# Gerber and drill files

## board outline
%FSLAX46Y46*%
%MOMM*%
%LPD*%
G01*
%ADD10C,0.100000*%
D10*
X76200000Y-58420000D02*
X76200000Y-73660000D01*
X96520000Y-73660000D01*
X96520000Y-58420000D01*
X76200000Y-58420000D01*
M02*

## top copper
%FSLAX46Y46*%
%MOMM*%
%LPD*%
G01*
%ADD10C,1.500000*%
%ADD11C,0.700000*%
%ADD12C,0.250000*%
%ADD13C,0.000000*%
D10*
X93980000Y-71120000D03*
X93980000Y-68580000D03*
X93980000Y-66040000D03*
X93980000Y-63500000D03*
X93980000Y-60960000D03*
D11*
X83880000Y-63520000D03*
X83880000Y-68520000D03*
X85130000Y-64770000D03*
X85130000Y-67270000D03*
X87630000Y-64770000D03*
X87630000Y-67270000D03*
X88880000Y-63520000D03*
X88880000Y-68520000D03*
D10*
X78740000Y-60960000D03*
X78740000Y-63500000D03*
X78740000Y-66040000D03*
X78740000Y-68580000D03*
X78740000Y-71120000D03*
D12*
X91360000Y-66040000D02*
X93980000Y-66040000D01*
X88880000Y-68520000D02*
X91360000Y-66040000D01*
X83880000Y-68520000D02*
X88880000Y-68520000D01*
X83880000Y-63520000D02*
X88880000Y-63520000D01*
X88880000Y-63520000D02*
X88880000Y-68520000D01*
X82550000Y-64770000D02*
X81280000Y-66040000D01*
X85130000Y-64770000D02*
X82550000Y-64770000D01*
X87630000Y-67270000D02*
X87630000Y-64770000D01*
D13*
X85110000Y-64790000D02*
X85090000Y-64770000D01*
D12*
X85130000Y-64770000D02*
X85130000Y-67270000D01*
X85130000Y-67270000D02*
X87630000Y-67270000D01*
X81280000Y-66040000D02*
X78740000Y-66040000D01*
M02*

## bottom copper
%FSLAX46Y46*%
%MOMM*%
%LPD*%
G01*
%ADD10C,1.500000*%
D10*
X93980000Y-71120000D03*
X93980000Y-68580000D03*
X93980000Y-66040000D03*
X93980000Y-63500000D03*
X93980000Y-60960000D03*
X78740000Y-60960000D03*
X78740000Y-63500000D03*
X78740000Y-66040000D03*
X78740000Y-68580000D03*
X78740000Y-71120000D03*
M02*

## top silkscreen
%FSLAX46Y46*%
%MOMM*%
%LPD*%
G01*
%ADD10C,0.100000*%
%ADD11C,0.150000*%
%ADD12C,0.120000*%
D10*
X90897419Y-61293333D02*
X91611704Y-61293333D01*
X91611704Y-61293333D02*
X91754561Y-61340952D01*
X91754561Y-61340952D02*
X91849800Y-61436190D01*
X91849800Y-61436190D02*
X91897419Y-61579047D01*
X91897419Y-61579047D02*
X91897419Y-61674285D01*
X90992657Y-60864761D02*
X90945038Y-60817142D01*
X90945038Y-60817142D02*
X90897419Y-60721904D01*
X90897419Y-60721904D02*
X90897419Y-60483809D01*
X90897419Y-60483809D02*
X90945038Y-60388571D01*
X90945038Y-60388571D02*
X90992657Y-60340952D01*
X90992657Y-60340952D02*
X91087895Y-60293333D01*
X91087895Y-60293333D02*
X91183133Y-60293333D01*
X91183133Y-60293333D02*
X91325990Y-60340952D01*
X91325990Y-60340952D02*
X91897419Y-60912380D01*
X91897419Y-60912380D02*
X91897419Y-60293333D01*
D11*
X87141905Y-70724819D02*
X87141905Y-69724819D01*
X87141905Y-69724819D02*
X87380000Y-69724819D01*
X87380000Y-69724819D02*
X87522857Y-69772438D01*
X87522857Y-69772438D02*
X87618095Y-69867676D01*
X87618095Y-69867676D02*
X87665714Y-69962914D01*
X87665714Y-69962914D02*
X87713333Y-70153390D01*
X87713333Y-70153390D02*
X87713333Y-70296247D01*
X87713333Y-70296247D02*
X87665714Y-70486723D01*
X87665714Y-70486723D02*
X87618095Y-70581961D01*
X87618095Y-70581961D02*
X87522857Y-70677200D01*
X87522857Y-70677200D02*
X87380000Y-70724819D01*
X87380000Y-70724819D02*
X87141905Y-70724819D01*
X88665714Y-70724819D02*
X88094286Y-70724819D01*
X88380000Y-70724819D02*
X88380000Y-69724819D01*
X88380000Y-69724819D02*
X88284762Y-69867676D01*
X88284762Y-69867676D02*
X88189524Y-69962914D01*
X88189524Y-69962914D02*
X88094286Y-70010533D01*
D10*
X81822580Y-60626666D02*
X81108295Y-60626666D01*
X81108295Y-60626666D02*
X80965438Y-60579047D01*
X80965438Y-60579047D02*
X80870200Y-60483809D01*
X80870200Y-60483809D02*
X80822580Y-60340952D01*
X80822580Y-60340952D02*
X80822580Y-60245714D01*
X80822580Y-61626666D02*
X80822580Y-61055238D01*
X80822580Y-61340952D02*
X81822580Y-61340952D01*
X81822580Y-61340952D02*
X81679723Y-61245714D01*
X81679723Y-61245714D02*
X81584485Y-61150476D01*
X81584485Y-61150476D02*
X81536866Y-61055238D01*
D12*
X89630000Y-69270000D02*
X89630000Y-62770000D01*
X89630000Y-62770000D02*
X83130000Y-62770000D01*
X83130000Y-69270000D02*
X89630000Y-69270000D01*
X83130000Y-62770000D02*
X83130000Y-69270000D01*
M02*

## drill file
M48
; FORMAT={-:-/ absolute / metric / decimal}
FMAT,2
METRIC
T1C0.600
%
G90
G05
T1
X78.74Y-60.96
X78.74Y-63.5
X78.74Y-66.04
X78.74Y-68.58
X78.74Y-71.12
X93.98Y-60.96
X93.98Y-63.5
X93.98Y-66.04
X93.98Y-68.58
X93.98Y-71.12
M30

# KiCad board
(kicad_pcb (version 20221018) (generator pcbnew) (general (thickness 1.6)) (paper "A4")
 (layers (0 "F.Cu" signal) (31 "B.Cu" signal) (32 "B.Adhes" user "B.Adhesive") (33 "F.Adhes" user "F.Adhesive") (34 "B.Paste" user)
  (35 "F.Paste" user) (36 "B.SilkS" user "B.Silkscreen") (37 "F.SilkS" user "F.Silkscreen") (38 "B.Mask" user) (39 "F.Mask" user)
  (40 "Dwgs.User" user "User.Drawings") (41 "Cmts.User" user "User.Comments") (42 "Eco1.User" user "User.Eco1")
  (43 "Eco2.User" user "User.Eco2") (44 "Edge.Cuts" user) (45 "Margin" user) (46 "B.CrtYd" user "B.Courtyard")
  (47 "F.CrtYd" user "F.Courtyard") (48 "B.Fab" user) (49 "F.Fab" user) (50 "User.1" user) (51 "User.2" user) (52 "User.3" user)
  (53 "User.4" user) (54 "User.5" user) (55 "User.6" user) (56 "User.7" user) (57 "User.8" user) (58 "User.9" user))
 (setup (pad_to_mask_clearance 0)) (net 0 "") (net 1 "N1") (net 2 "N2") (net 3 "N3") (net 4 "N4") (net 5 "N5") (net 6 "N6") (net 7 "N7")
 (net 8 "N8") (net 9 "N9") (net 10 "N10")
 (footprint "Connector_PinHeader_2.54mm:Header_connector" (layer "F.Cu") (at 93.98 66.04 90)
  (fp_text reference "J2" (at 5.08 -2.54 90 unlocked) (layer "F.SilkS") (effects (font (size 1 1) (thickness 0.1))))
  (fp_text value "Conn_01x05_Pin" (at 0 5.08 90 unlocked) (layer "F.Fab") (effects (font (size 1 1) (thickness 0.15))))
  (pad "1" thru_hole circle (at -5.08 0) (size 1.5 1.5) (drill 0.6) (layers "*.Cu" "*.Mask") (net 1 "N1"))
  (pad "2" thru_hole circle (at -2.54 0) (size 1.5 1.5) (drill 0.6) (layers "*.Cu" "*.Mask") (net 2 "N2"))
  (pad "3" thru_hole circle (at 0 0) (size 1.5 1.5) (drill 0.6) (layers "*.Cu" "*.Mask") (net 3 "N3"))
  (pad "4" thru_hole circle (at 2.54 0) (size 1.5 1.5) (drill 0.6) (layers "*.Cu" "*.Mask") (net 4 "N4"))
  (pad "5" thru_hole circle (at 5.08 0) (size 1.5 1.5) (drill 0.6) (layers "*.Cu" "*.Mask") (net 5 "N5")))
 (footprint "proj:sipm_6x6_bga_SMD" (layer "F.Cu") (at 83.88 63.52 180)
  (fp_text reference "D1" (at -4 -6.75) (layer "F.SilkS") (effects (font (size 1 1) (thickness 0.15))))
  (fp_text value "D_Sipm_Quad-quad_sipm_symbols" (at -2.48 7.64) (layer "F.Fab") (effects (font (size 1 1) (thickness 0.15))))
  (fp_line (start -5.75 -5.75) (end -5.75 0.75) (stroke (width 0.12) (type solid)) (layer "F.SilkS"))
  (fp_line (start -5.75 0.75) (end 0.75 0.75) (stroke (width 0.12) (type solid)) (layer "F.SilkS"))
  (fp_line (start 0.75 -5.75) (end -5.75 -5.75) (stroke (width 0.12) (type solid)) (layer "F.SilkS"))
  (fp_line (start 0.75 0.75) (end 0.75 -5.75) (stroke (width 0.12) (type solid)) (layer "F.SilkS"))
  (pad "A1" smd circle (at 0 0 180) (size 0.7 0.7) (layers "F.Cu" "F.Paste" "F.Mask") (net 3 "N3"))
  (pad "A4" smd circle (at 0 -5 180) (size 0.7 0.7) (layers "F.Cu" "F.Paste" "F.Mask") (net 3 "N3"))
  (pad "B2" smd circle (at -1.25 -1.25 180) (size 0.7 0.7) (layers "F.Cu" "F.Paste" "F.Mask") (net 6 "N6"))
  (pad "B3" smd circle (at -1.25 -3.75 180) (size 0.7 0.7) (layers "F.Cu" "F.Paste" "F.Mask") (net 6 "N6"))
  (pad "C2" smd circle (at -3.75 -1.25 180) (size 0.7 0.7) (layers "F.Cu" "F.Paste" "F.Mask") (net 6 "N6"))
  (pad "C3" smd circle (at -3.75 -3.75 180) (size 0.7 0.7) (layers "F.Cu" "F.Paste" "F.Mask") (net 6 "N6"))
  (pad "D1" smd circle (at -5 0 180) (size 0.7 0.7) (layers "F.Cu" "F.Paste" "F.Mask") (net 3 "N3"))
  (pad "D4" smd circle (at -5 -5 180) (size 0.7 0.7) (layers "F.Cu" "F.Paste" "F.Mask") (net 3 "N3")))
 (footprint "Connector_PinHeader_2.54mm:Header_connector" (layer "F.Cu") (at 78.74 66.04 -90)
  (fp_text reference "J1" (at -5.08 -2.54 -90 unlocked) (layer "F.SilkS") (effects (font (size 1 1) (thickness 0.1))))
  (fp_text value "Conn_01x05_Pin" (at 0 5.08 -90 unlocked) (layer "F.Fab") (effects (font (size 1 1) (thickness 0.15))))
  (pad "1" thru_hole circle (at -5.08 0 180) (size 1.5 1.5) (drill 0.6) (layers "*.Cu" "*.Mask") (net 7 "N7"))
  (pad "2" thru_hole circle (at -2.54 0 180) (size 1.5 1.5) (drill 0.6) (layers "*.Cu" "*.Mask") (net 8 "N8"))
  (pad "3" thru_hole circle (at 0 0 180) (size 1.5 1.5) (drill 0.6) (layers "*.Cu" "*.Mask") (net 6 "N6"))
  (pad "4" thru_hole circle (at 2.54 0 180) (size 1.5 1.5) (drill 0.6) (layers "*.Cu" "*.Mask") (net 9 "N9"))
  (pad "5" thru_hole circle (at 5.08 0 180) (size 1.5 1.5) (drill 0.6) (layers "*.Cu" "*.Mask") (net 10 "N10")))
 (gr_poly
  (pts (xy 76.2 58.42) (xy 76.2 73.66) (xy 96.52 73.66) (xy 96.52 58.42)) (stroke (width 0.1) (type solid)) (fill none) (layer "Edge.Cuts"))
 (segment (start 91.36 66.04) (end 93.98 66.04) (width 0.25) (layer "F.Cu") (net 3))
 (segment (start 88.88 68.52) (end 91.36 66.04) (width 0.25) (layer "F.Cu") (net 3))
 (segment (start 83.88 68.52) (end 88.88 68.52) (width 0.25) (layer "F.Cu") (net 3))
 (segment (start 83.88 63.52) (end 88.88 63.52) (width 0.25) (layer "F.Cu") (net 3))
 (segment (start 88.88 63.52) (end 88.88 68.52) (width 0.25) (layer "F.Cu") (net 3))
 (segment (start 82.55 64.77) (end 81.28 66.04) (width 0.25) (layer "F.Cu") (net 6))
 (segment (start 85.13 64.77) (end 82.55 64.77) (width 0.25) (layer "F.Cu") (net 6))
 (segment (start 87.63 67.27) (end 87.63 64.77) (width 0.25) (layer "F.Cu") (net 6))
 (segment (start 85.11 64.79) (end 85.09 64.77) (width 0) (layer "F.Cu") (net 6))
 (segment (start 85.13 64.77) (end 85.13 67.27) (width 0.25) (layer "F.Cu") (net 6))
 (segment (start 85.13 67.27) (end 87.63 67.27) (width 0.25) (layer "F.Cu") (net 6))
 (segment (start 81.28 66.04) (end 78.74 66.04) (width 0.25) (layer "F.Cu") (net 6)))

